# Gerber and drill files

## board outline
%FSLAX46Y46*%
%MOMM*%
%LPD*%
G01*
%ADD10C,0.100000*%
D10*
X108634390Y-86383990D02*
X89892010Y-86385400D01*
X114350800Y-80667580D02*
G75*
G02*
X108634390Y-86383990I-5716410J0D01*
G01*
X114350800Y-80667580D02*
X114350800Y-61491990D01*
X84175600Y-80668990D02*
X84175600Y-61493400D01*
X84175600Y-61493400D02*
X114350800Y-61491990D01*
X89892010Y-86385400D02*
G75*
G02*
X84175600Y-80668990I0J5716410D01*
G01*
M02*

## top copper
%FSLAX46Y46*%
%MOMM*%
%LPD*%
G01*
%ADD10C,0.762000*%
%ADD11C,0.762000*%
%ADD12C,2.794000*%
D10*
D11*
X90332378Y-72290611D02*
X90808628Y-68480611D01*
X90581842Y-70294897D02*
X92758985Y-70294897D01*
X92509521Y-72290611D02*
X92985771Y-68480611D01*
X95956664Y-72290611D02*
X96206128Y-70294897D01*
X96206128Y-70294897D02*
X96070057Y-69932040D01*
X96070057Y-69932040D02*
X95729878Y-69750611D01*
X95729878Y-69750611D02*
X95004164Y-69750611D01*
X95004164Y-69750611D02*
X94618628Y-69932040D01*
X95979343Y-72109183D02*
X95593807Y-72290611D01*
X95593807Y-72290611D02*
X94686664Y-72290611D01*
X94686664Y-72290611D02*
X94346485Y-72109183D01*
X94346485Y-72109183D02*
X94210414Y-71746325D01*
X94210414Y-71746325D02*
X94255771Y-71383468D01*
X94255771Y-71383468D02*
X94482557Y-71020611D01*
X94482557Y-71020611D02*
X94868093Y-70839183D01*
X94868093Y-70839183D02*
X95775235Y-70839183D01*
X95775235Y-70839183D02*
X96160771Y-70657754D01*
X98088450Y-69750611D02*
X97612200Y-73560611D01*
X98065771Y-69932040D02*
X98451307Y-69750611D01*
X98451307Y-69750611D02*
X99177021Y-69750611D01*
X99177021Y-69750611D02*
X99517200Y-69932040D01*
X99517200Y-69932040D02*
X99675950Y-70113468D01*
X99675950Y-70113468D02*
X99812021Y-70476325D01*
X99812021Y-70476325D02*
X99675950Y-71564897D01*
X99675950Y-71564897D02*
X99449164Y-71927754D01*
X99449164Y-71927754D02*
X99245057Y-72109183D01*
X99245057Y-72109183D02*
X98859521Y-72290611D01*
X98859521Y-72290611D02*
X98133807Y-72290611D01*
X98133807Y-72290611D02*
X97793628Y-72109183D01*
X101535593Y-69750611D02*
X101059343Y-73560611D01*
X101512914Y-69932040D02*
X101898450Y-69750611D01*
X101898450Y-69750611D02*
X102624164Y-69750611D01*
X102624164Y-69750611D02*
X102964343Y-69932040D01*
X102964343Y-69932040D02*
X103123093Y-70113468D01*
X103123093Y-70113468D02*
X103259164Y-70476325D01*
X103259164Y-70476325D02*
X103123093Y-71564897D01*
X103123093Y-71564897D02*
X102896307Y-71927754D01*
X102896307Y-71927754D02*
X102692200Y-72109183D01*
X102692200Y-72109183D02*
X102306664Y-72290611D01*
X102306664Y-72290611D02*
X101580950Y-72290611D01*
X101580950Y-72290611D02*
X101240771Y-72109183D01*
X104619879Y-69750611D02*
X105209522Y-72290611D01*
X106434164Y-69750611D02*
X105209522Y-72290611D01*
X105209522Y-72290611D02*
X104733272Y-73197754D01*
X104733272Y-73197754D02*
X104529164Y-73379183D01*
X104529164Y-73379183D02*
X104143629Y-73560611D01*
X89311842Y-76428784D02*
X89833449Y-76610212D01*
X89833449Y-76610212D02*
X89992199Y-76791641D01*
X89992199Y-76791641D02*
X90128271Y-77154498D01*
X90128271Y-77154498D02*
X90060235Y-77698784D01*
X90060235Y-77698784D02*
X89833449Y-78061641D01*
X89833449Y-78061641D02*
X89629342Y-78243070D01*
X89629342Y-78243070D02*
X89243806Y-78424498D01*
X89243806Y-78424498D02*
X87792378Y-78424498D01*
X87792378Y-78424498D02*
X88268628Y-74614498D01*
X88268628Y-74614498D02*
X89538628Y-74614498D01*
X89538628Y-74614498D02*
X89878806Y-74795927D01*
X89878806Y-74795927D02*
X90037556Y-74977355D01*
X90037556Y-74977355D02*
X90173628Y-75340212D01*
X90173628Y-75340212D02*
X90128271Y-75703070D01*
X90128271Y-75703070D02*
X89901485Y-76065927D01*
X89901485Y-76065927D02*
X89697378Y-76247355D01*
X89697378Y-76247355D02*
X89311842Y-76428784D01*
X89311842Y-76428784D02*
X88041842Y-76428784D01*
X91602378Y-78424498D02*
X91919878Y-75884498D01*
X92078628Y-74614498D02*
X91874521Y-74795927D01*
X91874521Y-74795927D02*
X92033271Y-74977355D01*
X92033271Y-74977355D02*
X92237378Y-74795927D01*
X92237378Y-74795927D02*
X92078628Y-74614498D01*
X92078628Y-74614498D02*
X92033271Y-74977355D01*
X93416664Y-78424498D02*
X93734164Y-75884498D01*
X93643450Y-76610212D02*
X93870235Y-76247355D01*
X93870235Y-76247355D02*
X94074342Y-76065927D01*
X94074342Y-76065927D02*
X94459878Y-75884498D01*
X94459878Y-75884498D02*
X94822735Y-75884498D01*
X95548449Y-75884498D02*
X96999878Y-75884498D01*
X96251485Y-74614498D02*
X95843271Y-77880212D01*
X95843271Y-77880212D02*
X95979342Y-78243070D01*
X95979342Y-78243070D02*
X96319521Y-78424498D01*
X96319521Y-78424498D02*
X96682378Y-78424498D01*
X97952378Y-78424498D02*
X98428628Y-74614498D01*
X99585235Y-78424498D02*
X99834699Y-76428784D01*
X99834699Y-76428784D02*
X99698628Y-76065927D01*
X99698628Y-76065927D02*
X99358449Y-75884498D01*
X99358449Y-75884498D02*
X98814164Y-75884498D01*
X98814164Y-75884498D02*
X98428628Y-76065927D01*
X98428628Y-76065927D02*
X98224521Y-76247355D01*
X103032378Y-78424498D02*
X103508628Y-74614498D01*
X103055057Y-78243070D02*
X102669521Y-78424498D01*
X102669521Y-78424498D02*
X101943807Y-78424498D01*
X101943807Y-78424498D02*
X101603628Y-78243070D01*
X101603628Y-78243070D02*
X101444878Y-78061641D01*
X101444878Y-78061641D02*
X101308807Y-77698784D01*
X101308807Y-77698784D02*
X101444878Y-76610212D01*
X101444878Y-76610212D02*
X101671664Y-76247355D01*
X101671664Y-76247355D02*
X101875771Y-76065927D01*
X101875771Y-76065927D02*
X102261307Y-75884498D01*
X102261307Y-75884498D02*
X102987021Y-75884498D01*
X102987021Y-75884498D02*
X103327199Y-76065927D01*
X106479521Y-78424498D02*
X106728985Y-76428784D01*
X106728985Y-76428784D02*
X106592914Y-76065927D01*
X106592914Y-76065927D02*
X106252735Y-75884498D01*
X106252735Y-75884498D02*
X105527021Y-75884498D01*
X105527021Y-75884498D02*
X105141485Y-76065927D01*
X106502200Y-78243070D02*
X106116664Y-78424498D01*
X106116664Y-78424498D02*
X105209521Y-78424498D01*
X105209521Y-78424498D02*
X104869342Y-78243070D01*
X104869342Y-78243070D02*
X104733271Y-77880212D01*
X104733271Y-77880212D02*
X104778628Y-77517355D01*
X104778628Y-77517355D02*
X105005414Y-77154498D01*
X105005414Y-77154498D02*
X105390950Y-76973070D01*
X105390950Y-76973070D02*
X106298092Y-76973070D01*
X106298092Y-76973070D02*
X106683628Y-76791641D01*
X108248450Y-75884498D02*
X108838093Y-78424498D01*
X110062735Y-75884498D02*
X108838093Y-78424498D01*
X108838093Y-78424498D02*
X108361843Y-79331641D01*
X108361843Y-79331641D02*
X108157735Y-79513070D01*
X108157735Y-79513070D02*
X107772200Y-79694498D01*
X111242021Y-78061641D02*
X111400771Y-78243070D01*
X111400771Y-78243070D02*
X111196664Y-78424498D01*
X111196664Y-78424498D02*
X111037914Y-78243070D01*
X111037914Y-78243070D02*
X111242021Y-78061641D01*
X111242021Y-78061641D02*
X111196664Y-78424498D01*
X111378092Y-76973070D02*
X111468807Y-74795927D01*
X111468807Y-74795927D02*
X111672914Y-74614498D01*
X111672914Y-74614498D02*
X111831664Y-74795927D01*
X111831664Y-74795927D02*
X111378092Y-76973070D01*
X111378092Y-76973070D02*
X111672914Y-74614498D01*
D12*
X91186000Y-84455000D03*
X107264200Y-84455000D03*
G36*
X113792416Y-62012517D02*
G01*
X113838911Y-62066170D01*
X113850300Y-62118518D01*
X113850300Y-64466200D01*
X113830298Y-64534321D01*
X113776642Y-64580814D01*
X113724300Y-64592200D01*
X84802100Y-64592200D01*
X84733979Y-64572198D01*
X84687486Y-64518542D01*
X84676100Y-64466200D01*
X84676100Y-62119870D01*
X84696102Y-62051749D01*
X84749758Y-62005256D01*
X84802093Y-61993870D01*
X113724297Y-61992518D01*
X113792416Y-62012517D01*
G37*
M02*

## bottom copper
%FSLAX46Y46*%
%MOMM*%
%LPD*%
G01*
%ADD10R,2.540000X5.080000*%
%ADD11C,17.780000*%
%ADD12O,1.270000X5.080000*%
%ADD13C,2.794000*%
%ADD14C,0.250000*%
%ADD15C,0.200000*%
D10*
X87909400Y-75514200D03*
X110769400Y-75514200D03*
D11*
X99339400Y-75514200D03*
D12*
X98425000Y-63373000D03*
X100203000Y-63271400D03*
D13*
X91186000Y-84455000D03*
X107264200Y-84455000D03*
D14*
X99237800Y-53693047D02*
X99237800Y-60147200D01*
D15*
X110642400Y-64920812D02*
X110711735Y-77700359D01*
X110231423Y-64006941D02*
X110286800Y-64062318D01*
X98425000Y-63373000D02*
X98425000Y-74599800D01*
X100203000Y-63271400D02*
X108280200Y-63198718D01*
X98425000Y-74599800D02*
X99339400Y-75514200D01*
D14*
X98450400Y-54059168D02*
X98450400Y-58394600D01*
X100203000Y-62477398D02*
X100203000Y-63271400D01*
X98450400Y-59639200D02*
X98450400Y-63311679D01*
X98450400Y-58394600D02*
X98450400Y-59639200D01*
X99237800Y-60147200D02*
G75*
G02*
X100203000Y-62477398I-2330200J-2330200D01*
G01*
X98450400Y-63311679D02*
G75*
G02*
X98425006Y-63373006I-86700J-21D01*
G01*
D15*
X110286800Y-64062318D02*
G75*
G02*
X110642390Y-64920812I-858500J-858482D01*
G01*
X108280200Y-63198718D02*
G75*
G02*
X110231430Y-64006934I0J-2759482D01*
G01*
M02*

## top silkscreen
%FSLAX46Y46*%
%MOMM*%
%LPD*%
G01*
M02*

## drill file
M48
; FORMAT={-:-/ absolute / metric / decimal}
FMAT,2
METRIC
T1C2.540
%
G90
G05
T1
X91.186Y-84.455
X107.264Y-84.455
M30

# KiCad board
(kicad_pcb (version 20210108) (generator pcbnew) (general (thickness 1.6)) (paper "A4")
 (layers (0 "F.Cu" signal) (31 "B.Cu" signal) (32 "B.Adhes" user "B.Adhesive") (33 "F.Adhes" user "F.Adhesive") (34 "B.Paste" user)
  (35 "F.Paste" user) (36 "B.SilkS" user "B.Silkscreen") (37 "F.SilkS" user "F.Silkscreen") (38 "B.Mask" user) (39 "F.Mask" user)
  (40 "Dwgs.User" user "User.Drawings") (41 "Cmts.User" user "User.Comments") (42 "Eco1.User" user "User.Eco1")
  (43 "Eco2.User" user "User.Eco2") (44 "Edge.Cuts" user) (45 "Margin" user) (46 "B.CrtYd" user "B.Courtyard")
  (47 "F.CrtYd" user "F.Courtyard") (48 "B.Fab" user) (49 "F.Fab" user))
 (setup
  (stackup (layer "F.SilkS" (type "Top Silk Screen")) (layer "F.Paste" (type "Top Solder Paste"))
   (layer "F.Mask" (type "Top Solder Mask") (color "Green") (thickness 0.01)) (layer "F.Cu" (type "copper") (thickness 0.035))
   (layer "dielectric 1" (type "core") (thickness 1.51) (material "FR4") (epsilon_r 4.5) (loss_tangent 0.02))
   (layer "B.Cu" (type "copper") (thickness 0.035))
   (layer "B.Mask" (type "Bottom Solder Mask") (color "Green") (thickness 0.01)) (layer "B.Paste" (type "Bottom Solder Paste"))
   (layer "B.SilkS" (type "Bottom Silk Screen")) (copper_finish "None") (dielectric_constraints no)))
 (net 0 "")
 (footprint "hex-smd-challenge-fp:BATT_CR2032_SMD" (layer "B.Cu") (at 99.3394 75.5142 180)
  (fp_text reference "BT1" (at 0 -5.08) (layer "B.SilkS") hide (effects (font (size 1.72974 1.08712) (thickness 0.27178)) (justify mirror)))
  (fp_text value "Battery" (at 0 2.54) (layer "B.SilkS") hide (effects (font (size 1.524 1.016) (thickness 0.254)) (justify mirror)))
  (pad "1" smd rect (at 11.43 0 180) (locked) (size 2.54 5.08) (layers "B.Cu" "B.Paste" "B.Mask"))
  (pad "1" smd rect (at -11.43 0 180) (locked) (size 2.54 5.08) (layers "B.Cu" "B.Paste" "B.Mask"))
  (pad "2" smd circle (at 0 0 180) (locked) (size 17.78 17.78) (layers "B.Cu" "B.Paste" "B.Mask")))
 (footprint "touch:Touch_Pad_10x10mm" (layer "B.Cu") (at 98.7552 63.1952)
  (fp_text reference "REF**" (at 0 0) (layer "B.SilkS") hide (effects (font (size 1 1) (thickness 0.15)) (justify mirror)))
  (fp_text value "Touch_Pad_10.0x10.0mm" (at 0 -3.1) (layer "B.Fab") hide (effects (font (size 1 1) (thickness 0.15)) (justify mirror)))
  (pad "1" smd oval (at -0.3302 0.1778) (locked) (size 1.27 5.08) (layers "B.Cu" "B.Mask")))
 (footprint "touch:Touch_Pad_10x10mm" (layer "B.Cu") (at 100.5332 63.0936)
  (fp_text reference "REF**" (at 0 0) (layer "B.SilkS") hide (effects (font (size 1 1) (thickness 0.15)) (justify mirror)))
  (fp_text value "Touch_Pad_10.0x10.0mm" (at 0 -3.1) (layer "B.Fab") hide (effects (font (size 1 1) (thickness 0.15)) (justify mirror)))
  (pad "1" smd oval (at -0.3302 0.1778) (locked) (size 1.27 5.08) (layers "B.Cu" "B.Mask")))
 (gr_line (start 108.63439 86.38399) (end 89.89201 86.3854) (layer "Edge.Cuts") (width 0.1))
 (gr_arc (start 108.63439 80.66758) (end 114.3508 80.66758) (angle 90) (layer "Edge.Cuts") (width 0.1))
 (gr_line (start 114.3508 80.66758) (end 114.3508 61.49199) (layer "Edge.Cuts") (width 0.1))
 (gr_line (start 84.1756 80.66899) (end 84.1756 61.4934) (layer "Edge.Cuts") (width 0.1))
 (gr_line (start 84.1756 61.4934) (end 114.3508 61.49199) (layer "Edge.Cuts") (width 0.1))
 (gr_arc (start 89.89201 80.66899) (end 84.1756 80.66899) (angle -90) (layer "Edge.Cuts") (width 0.1))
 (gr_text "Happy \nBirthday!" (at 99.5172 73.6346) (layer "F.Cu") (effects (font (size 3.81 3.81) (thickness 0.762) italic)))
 (via (at 91.186 84.455) (size 2.794) (drill 2.54) (layers "F.Cu" "B.Cu") (free) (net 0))
 (via (at 107.2642 84.455) (size 2.794) (drill 2.54) (layers "F.Cu" "B.Cu") (free) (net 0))
 (segment (start 99.2378 53.693047) (end 99.2378 60.1472) (width 0.25) (layer "B.Cu") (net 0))
 (segment (start 110.6424 64.920812) (end 110.711735 77.700359) (width 0.2) (layer "B.Cu") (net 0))
 (segment (start 110.231423 64.006941) (end 110.2868 64.062318) (width 0.2) (layer "B.Cu") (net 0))
 (segment (start 98.425 63.373) (end 98.425 74.5998) (width 0.2) (layer "B.Cu") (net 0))
 (segment (start 100.203 63.2714) (end 108.2802 63.198718) (width 0.2) (layer "B.Cu") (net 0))
 (segment (start 98.425 74.5998) (end 99.3394 75.5142) (width 0.2) (layer "B.Cu") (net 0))
 (segment (start 98.4504 54.059168) (end 98.4504 58.3946) (width 0.25) (layer "B.Cu") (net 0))
 (segment (start 100.203 62.477398) (end 100.203 63.2714) (width 0.25) (layer "B.Cu") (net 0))
 (segment (start 98.4504 59.6392) (end 98.4504 63.311679) (width 0.25) (layer "B.Cu") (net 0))
 (segment (start 98.4504 58.3946) (end 98.4504 59.6392) (width 0.25) (layer "B.Cu") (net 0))
 (arc (start 99.2378 60.1472) (mid 99.952152 61.216303) (end 100.203 62.477398) (width 0.25) (layer "B.Cu") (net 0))
 (arc (start 98.4504 63.311679) (mid 98.443799 63.344864) (end 98.425 63.373) (width 0.25) (layer "B.Cu") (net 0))
 (arc (start 110.2868 64.062318) (mid 110.549983 64.456198) (end 110.6424 64.920812) (width 0.2) (layer "B.Cu") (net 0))
 (arc (start 108.2802 63.198718) (mid 109.336194 63.408768) (end 110.231423 64.006941) (width 0.2) (layer "B.Cu") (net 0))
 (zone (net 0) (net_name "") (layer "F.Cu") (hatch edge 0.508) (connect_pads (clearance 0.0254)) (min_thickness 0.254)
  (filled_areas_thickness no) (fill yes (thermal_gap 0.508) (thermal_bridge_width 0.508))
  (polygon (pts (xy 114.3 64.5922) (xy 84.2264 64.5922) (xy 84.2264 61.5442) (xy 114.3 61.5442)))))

